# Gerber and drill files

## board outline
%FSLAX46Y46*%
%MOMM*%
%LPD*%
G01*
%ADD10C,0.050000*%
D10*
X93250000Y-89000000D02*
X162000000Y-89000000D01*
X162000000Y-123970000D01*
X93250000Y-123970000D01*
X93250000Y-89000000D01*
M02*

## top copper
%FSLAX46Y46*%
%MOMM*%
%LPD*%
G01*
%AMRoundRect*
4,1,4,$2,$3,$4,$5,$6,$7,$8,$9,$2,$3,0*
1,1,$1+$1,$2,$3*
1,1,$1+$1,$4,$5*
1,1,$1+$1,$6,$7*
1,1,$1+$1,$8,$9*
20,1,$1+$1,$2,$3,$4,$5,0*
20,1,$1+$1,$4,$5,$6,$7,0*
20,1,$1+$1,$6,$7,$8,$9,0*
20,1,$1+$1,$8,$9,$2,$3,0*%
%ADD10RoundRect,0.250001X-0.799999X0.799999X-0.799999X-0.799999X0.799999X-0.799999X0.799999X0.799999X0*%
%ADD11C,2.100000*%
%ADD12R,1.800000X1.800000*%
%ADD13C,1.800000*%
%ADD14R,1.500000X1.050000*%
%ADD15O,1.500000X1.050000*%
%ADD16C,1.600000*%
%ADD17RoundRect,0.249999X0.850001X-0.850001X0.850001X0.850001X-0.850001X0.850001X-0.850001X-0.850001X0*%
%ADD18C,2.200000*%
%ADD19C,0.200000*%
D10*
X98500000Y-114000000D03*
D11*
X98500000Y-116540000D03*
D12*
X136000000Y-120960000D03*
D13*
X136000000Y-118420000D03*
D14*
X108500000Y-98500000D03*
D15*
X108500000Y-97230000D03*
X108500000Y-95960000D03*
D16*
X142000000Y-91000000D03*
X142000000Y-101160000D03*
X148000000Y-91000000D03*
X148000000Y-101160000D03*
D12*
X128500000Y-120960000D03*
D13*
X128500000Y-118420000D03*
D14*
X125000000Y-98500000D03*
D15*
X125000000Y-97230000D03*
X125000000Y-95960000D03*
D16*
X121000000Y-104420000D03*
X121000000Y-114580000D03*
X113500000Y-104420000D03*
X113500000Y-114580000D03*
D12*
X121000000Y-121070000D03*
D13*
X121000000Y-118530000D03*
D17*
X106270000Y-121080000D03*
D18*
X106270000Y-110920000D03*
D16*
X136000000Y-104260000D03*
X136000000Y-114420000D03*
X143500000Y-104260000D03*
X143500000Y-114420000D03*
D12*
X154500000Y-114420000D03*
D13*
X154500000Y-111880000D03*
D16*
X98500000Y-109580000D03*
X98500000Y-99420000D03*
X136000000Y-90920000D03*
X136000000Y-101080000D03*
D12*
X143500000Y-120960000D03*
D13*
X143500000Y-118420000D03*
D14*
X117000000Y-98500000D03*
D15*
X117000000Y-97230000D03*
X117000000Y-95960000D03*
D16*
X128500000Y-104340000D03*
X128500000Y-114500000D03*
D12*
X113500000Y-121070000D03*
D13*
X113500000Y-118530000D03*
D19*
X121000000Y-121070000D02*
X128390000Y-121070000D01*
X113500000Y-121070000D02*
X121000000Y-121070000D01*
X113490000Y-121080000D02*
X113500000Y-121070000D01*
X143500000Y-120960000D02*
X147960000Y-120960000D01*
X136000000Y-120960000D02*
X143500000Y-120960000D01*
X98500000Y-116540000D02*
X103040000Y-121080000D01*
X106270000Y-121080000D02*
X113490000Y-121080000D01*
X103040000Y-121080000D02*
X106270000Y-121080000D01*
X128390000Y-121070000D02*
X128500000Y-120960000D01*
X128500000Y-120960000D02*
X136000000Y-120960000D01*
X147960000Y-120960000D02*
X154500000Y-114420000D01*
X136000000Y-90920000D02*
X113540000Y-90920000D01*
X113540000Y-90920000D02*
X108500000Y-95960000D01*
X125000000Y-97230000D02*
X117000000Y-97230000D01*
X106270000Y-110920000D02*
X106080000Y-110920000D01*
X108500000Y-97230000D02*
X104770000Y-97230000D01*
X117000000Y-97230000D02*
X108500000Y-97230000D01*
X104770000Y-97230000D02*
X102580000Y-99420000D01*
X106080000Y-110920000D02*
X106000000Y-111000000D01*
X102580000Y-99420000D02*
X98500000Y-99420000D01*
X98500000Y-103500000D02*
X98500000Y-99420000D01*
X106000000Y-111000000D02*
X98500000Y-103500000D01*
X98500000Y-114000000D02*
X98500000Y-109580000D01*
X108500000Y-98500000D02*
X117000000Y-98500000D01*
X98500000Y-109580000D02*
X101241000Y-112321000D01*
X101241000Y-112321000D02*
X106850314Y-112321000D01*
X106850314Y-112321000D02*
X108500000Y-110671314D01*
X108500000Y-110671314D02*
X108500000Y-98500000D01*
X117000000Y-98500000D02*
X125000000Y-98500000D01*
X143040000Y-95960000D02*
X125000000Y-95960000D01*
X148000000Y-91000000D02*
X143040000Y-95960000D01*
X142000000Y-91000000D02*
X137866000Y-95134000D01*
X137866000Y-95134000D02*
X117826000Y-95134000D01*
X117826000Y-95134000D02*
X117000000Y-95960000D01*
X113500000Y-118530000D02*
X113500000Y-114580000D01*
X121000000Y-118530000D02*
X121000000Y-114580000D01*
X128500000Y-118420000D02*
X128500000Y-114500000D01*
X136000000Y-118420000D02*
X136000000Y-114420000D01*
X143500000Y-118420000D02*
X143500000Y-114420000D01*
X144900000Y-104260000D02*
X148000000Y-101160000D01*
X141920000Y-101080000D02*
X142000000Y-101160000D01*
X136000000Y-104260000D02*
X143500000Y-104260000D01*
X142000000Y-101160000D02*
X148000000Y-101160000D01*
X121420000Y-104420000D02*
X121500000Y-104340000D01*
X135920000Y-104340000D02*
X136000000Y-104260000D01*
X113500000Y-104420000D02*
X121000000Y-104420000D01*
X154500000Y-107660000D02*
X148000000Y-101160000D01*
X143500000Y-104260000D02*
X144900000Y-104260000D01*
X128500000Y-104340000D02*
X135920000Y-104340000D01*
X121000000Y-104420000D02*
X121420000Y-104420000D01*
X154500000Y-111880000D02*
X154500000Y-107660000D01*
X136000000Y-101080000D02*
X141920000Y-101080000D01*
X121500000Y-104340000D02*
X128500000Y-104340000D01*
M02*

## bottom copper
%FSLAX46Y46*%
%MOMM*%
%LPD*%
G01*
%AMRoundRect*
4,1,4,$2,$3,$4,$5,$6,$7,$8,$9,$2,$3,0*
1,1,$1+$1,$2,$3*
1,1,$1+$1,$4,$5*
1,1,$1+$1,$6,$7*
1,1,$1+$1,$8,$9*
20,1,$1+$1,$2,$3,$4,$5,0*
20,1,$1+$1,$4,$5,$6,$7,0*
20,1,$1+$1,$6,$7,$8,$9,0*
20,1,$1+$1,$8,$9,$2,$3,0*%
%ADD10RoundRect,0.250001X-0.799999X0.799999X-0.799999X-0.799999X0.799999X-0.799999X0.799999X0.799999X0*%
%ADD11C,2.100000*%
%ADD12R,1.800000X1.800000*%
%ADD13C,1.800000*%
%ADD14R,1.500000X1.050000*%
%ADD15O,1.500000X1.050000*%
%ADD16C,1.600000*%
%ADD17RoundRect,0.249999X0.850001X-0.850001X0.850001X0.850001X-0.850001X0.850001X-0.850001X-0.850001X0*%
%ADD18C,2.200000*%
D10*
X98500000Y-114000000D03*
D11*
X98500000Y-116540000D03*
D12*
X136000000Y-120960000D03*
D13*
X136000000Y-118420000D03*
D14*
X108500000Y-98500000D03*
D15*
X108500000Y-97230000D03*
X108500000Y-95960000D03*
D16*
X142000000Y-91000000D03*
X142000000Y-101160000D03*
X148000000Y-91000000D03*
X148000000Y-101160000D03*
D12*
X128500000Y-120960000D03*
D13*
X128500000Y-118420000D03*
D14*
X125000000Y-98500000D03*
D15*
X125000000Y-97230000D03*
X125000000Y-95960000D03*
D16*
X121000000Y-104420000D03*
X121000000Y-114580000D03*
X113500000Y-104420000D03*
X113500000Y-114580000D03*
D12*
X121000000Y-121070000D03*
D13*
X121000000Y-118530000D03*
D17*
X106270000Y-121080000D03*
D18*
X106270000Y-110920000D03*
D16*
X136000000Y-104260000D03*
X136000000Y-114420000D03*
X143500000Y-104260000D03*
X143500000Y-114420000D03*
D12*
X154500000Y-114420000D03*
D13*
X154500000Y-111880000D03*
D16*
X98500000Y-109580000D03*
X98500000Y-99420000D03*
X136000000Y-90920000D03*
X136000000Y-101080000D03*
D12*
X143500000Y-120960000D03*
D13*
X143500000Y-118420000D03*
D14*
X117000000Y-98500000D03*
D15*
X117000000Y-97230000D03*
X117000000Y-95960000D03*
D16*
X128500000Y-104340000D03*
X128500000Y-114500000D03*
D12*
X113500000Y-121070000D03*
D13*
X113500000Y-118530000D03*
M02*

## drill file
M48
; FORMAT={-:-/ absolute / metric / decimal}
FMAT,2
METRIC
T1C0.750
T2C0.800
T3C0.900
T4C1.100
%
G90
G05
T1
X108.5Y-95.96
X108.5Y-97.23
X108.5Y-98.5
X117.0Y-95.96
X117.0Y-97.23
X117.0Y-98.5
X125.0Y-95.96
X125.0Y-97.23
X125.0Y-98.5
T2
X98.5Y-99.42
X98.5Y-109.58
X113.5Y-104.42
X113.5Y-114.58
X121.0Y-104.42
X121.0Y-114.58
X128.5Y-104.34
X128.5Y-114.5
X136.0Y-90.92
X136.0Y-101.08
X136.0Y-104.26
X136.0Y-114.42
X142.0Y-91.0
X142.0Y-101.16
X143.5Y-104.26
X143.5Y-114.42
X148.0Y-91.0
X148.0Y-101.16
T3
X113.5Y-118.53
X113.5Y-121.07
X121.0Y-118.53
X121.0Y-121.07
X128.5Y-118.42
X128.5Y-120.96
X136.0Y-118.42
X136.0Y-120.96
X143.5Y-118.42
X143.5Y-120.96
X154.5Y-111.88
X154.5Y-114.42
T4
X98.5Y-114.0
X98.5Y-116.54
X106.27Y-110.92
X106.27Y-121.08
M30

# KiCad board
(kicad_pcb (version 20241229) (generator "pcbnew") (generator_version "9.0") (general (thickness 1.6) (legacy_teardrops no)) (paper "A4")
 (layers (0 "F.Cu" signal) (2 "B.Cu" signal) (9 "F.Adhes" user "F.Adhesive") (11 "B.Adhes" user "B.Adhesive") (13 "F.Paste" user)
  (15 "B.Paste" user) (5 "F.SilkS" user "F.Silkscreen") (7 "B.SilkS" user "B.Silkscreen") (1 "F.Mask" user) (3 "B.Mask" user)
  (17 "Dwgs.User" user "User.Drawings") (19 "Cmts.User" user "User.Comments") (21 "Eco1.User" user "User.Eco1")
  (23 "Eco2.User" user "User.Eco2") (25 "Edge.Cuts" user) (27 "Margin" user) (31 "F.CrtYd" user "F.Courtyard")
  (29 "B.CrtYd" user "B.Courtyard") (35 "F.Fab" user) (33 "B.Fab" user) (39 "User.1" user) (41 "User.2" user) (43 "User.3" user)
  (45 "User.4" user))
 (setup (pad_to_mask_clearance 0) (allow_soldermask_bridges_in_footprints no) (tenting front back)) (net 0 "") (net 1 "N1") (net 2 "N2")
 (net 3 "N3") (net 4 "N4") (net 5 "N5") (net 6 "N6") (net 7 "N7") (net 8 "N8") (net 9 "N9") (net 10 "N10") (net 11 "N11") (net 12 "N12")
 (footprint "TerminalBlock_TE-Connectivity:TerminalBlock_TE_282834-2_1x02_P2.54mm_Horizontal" (layer "F.Cu") (at 98.5 114 -90)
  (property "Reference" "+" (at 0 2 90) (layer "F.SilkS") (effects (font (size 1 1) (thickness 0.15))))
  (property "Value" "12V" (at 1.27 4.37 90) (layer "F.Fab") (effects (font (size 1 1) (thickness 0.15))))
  (pad "1" thru_hole roundrect (at 0 0 270) (size 2.1 2.1) (drill 1.1) (layers "*.Cu" "*.Mask") (remove_unused_layers no)
   (roundrect_rratio 0.119048) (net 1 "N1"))
  (pad "2" thru_hole circle (at 2.54 0 270) (size 2.1 2.1) (drill 1.1) (layers "*.Cu" "*.Mask") (remove_unused_layers no) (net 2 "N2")))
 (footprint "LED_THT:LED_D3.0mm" (layer "F.Cu") (at 136 120.96 90)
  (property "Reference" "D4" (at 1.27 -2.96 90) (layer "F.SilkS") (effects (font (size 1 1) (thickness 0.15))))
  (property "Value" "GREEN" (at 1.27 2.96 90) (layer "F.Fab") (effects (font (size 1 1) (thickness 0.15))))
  (pad "1" thru_hole rect (at 0 0 90) (size 1.8 1.8) (drill 0.9) (layers "*.Cu" "*.Mask") (remove_unused_layers no) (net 2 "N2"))
  (pad "2" thru_hole circle (at 2.54 0 90) (size 1.8 1.8) (drill 0.9) (layers "*.Cu" "*.Mask") (remove_unused_layers no) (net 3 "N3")))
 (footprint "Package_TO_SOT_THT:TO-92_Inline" (layer "F.Cu") (at 108.5 98.5 90)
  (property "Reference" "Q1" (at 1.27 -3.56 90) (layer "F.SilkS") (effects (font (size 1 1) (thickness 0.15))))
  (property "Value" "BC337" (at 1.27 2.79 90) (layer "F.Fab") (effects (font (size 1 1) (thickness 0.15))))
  (pad "1" thru_hole rect (at 0 0 90) (size 1.05 1.5) (drill 0.75) (layers "*.Cu" "*.Mask") (remove_unused_layers no) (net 1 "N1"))
  (pad "2" thru_hole oval (at 1.27 0 90) (size 1.05 1.5) (drill 0.75) (layers "*.Cu" "*.Mask") (remove_unused_layers no) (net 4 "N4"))
  (pad "3" thru_hole oval (at 2.54 0 90) (size 1.05 1.5) (drill 0.75) (layers "*.Cu" "*.Mask") (remove_unused_layers no) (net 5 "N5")))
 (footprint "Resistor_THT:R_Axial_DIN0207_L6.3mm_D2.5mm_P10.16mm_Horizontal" (layer "F.Cu") (at 142 91 -90)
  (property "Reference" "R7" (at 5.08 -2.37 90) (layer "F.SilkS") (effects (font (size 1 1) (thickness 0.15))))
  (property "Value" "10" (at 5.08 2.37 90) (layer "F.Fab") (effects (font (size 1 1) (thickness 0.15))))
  (pad "1" thru_hole circle (at 0 0 270) (size 1.6 1.6) (drill 0.8) (layers "*.Cu" "*.Mask") (remove_unused_layers no) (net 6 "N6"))
  (pad "2" thru_hole circle (at 10.16 0 270) (size 1.6 1.6) (drill 0.8) (layers "*.Cu" "*.Mask") (remove_unused_layers no) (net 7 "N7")))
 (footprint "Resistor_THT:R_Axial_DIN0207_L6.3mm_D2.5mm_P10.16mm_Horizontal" (layer "F.Cu") (at 148 91 -90)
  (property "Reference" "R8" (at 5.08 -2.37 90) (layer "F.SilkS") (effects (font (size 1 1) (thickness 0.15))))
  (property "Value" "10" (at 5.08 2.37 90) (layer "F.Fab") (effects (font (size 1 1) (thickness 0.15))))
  (pad "1" thru_hole circle (at 0 0 270) (size 1.6 1.6) (drill 0.8) (layers "*.Cu" "*.Mask") (remove_unused_layers no) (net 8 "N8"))
  (pad "2" thru_hole circle (at 10.16 0 270) (size 1.6 1.6) (drill 0.8) (layers "*.Cu" "*.Mask") (remove_unused_layers no) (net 7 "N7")))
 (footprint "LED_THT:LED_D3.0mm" (layer "F.Cu") (at 128.5 120.96 90)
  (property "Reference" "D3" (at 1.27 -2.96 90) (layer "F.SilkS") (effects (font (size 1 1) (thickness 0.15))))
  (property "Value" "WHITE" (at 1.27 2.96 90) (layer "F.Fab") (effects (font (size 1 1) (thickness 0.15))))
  (pad "1" thru_hole rect (at 0 0 90) (size 1.8 1.8) (drill 0.9) (layers "*.Cu" "*.Mask") (remove_unused_layers no) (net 2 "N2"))
  (pad "2" thru_hole circle (at 2.54 0 90) (size 1.8 1.8) (drill 0.9) (layers "*.Cu" "*.Mask") (remove_unused_layers no) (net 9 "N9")))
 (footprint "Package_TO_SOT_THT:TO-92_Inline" (layer "F.Cu") (at 125 98.5 90)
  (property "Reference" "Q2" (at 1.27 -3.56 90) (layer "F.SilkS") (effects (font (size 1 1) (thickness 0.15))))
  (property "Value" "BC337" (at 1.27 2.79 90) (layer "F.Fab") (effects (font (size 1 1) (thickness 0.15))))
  (pad "1" thru_hole rect (at 0 0 90) (size 1.05 1.5) (drill 0.75) (layers "*.Cu" "*.Mask") (remove_unused_layers no) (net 1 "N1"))
  (pad "2" thru_hole oval (at 1.27 0 90) (size 1.05 1.5) (drill 0.75) (layers "*.Cu" "*.Mask") (remove_unused_layers no) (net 4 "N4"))
  (pad "3" thru_hole oval (at 2.54 0 90) (size 1.05 1.5) (drill 0.75) (layers "*.Cu" "*.Mask") (remove_unused_layers no) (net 8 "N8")))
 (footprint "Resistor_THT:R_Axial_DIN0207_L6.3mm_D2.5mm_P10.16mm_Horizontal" (layer "F.Cu") (at 121 104.42 -90)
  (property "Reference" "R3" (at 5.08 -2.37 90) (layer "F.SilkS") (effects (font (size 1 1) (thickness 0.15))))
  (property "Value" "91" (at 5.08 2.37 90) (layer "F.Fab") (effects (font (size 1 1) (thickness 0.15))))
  (pad "1" thru_hole circle (at 0 0 270) (size 1.6 1.6) (drill 0.8) (layers "*.Cu" "*.Mask") (remove_unused_layers no) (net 7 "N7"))
  (pad "2" thru_hole circle (at 10.16 0 270) (size 1.6 1.6) (drill 0.8) (layers "*.Cu" "*.Mask") (remove_unused_layers no) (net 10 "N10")))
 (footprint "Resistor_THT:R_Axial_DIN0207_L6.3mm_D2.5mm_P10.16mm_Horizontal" (layer "F.Cu") (at 113.5 104.42 -90)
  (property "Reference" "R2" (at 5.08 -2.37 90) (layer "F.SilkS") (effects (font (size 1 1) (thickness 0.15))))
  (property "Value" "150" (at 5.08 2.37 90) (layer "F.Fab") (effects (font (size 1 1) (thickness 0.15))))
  (pad "1" thru_hole circle (at 0 0 270) (size 1.6 1.6) (drill 0.8) (layers "*.Cu" "*.Mask") (remove_unused_layers no) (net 7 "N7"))
  (pad "2" thru_hole circle (at 10.16 0 270) (size 1.6 1.6) (drill 0.8) (layers "*.Cu" "*.Mask") (remove_unused_layers no) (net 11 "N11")))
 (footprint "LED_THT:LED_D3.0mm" (layer "F.Cu") (at 121 121.07 90)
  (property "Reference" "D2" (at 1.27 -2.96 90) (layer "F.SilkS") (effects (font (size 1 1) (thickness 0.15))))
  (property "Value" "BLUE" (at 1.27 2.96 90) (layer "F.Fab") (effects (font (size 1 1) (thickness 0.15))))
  (pad "1" thru_hole rect (at 0 0 90) (size 1.8 1.8) (drill 0.9) (layers "*.Cu" "*.Mask") (remove_unused_layers no) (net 2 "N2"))
  (pad "2" thru_hole circle (at 2.54 0 90) (size 1.8 1.8) (drill 0.9) (layers "*.Cu" "*.Mask") (remove_unused_layers no) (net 10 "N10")))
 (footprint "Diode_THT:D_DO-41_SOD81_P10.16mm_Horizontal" (layer "F.Cu") (at 106.27 121.08 90)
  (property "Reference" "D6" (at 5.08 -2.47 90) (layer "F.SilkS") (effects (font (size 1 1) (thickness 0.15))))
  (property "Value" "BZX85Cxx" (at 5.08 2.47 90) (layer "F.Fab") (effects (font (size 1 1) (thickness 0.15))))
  (pad "1" thru_hole roundrect (at 0 0 90) (size 2.2 2.2) (drill 1.1) (layers "*.Cu" "*.Mask") (remove_unused_layers no)
   (roundrect_rratio 0.113636) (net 2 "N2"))
  (pad "2" thru_hole circle (at 10.16 0 90) (size 2.2 2.2) (drill 1.1) (layers "*.Cu" "*.Mask") (remove_unused_layers no) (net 4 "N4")))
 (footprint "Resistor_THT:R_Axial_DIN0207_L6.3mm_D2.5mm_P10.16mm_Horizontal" (layer "F.Cu") (at 136 104.26 -90)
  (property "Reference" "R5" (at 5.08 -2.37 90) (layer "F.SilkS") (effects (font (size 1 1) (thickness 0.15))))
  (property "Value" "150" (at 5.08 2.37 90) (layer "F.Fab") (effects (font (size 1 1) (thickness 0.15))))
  (pad "1" thru_hole circle (at 0 0 270) (size 1.6 1.6) (drill 0.8) (layers "*.Cu" "*.Mask") (remove_unused_layers no) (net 7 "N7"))
  (pad "2" thru_hole circle (at 10.16 0 270) (size 1.6 1.6) (drill 0.8) (layers "*.Cu" "*.Mask") (remove_unused_layers no) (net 3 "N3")))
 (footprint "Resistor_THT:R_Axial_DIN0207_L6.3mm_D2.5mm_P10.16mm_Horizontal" (layer "F.Cu") (at 143.5 104.26 -90)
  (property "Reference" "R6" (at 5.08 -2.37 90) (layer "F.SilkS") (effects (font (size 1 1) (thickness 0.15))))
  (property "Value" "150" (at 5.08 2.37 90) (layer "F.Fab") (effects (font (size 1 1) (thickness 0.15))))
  (pad "1" thru_hole circle (at 0 0 270) (size 1.6 1.6) (drill 0.8) (layers "*.Cu" "*.Mask") (remove_unused_layers no) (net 7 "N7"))
  (pad "2" thru_hole circle (at 10.16 0 270) (size 1.6 1.6) (drill 0.8) (layers "*.Cu" "*.Mask") (remove_unused_layers no) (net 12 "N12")))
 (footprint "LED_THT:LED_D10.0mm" (layer "F.Cu") (at 154.5 114.42 90)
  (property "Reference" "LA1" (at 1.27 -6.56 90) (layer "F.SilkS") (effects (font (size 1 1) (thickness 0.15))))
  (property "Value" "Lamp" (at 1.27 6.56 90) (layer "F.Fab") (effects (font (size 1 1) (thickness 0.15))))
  (pad "1" thru_hole rect (at 0 0 90) (size 1.8 1.8) (drill 0.9) (layers "*.Cu" "*.Mask") (remove_unused_layers no) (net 2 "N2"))
  (pad "2" thru_hole circle (at 2.54 0 90) (size 1.8 1.8) (drill 0.9) (layers "*.Cu" "*.Mask") (remove_unused_layers no) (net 7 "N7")))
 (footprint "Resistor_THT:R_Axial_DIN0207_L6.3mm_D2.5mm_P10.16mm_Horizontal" (layer "F.Cu") (at 98.5 109.58 90)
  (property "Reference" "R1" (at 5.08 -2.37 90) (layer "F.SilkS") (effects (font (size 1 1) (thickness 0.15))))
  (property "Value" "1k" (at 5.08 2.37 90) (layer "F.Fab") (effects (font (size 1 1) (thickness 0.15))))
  (pad "1" thru_hole circle (at 0 0 90) (size 1.6 1.6) (drill 0.8) (layers "*.Cu" "*.Mask") (remove_unused_layers no) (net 1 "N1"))
  (pad "2" thru_hole circle (at 10.16 0 90) (size 1.6 1.6) (drill 0.8) (layers "*.Cu" "*.Mask") (remove_unused_layers no) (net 4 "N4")))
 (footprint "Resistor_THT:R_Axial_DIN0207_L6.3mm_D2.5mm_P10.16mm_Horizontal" (layer "F.Cu") (at 136 90.92 -90)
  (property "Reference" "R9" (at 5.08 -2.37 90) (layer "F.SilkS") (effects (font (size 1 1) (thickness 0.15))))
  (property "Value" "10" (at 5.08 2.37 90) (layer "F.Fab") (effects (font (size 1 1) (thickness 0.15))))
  (pad "1" thru_hole circle (at 0 0 270) (size 1.6 1.6) (drill 0.8) (layers "*.Cu" "*.Mask") (remove_unused_layers no) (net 5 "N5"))
  (pad "2" thru_hole circle (at 10.16 0 270) (size 1.6 1.6) (drill 0.8) (layers "*.Cu" "*.Mask") (remove_unused_layers no) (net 7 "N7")))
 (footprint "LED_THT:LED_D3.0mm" (layer "F.Cu") (at 143.5 120.96 90)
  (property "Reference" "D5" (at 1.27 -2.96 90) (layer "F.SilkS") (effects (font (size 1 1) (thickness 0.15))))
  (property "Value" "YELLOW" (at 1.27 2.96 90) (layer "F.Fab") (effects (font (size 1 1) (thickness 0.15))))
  (pad "1" thru_hole rect (at 0 0 90) (size 1.8 1.8) (drill 0.9) (layers "*.Cu" "*.Mask") (remove_unused_layers no) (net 2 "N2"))
  (pad "2" thru_hole circle (at 2.54 0 90) (size 1.8 1.8) (drill 0.9) (layers "*.Cu" "*.Mask") (remove_unused_layers no) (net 12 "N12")))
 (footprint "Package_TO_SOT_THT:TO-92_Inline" (layer "F.Cu") (at 117 98.5 90)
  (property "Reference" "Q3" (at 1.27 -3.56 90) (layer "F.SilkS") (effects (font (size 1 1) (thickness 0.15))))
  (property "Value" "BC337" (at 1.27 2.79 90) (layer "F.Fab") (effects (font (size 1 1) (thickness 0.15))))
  (pad "1" thru_hole rect (at 0 0 90) (size 1.05 1.5) (drill 0.75) (layers "*.Cu" "*.Mask") (remove_unused_layers no) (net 1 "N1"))
  (pad "2" thru_hole oval (at 1.27 0 90) (size 1.05 1.5) (drill 0.75) (layers "*.Cu" "*.Mask") (remove_unused_layers no) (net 4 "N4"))
  (pad "3" thru_hole oval (at 2.54 0 90) (size 1.05 1.5) (drill 0.75) (layers "*.Cu" "*.Mask") (remove_unused_layers no) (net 6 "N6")))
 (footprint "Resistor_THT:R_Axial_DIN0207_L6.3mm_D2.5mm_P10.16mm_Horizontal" (layer "F.Cu") (at 128.5 104.34 -90)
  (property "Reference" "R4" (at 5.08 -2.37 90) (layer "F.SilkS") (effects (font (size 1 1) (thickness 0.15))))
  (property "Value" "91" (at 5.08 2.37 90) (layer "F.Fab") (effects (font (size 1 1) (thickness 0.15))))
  (pad "1" thru_hole circle (at 0 0 270) (size 1.6 1.6) (drill 0.8) (layers "*.Cu" "*.Mask") (remove_unused_layers no) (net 7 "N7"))
  (pad "2" thru_hole circle (at 10.16 0 270) (size 1.6 1.6) (drill 0.8) (layers "*.Cu" "*.Mask") (remove_unused_layers no) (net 9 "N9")))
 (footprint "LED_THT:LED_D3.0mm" (layer "F.Cu") (at 113.5 121.07 90)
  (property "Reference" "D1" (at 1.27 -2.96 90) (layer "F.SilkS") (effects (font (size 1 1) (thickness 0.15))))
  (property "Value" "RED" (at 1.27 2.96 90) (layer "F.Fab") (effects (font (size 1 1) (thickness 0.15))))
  (pad "1" thru_hole rect (at 0 0 90) (size 1.8 1.8) (drill 0.9) (layers "*.Cu" "*.Mask") (remove_unused_layers no) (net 2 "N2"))
  (pad "2" thru_hole circle (at 2.54 0 90) (size 1.8 1.8) (drill 0.9) (layers "*.Cu" "*.Mask") (remove_unused_layers no) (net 11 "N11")))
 (gr_rect (start 93.25 89) (end 162 123.97) (stroke (width 0.05) (type default)) (fill no) (layer "Edge.Cuts"))
 (segment (start 121 121.07) (end 128.39 121.07) (width 0.2) (layer "F.Cu") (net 2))
 (segment (start 113.5 121.07) (end 121 121.07) (width 0.2) (layer "F.Cu") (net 2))
 (segment (start 113.49 121.08) (end 113.5 121.07) (width 0.2) (layer "F.Cu") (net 2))
 (segment (start 143.5 120.96) (end 147.96 120.96) (width 0.2) (layer "F.Cu") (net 2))
 (segment (start 136 120.96) (end 143.5 120.96) (width 0.2) (layer "F.Cu") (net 2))
 (segment (start 98.5 116.54) (end 103.04 121.08) (width 0.2) (layer "F.Cu") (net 2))
 (segment (start 106.27 121.08) (end 113.49 121.08) (width 0.2) (layer "F.Cu") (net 2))
 (segment (start 103.04 121.08) (end 106.27 121.08) (width 0.2) (layer "F.Cu") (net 2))
 (segment (start 128.39 121.07) (end 128.5 120.96) (width 0.2) (layer "F.Cu") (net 2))
 (segment (start 128.5 120.96) (end 136 120.96) (width 0.2) (layer "F.Cu") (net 2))
 (segment (start 147.96 120.96) (end 154.5 114.42) (width 0.2) (layer "F.Cu") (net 2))
 (segment (start 136 90.92) (end 113.54 90.92) (width 0.2) (layer "F.Cu") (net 5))
 (segment (start 113.54 90.92) (end 108.5 95.96) (width 0.2) (layer "F.Cu") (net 5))
 (segment (start 125 97.23) (end 117 97.23) (width 0.2) (layer "F.Cu") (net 4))
 (segment (start 106.27 110.92) (end 106.08 110.92) (width 0.2) (layer "F.Cu") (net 4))
 (segment (start 108.5 97.23) (end 104.77 97.23) (width 0.2) (layer "F.Cu") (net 4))
 (segment (start 117 97.23) (end 108.5 97.23) (width 0.2) (layer "F.Cu") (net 4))
 (segment (start 104.77 97.23) (end 102.58 99.42) (width 0.2) (layer "F.Cu") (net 4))
 (segment (start 106.08 110.92) (end 106 111) (width 0.2) (layer "F.Cu") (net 4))
 (segment (start 102.58 99.42) (end 98.5 99.42) (width 0.2) (layer "F.Cu") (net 4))
 (segment (start 98.5 103.5) (end 98.5 99.42) (width 0.2) (layer "F.Cu") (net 4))
 (segment (start 106 111) (end 98.5 103.5) (width 0.2) (layer "F.Cu") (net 4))
 (segment (start 98.5 114) (end 98.5 109.58) (width 0.2) (layer "F.Cu") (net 1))
 (segment (start 108.5 98.5) (end 117 98.5) (width 0.2) (layer "F.Cu") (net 1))
 (segment (start 98.5 109.58) (end 101.241 112.321) (width 0.2) (layer "F.Cu") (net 1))
 (segment (start 101.241 112.321) (end 106.850314 112.321) (width 0.2) (layer "F.Cu") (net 1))
 (segment (start 106.850314 112.321) (end 108.5 110.671314) (width 0.2) (layer "F.Cu") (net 1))
 (segment (start 108.5 110.671314) (end 108.5 98.5) (width 0.2) (layer "F.Cu") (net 1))
 (segment (start 117 98.5) (end 125 98.5) (width 0.2) (layer "F.Cu") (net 1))
 (segment (start 143.04 95.96) (end 125 95.96) (width 0.2) (layer "F.Cu") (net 8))
 (segment (start 148 91) (end 143.04 95.96) (width 0.2) (layer "F.Cu") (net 8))
 (segment (start 142 91) (end 137.866 95.134) (width 0.2) (layer "F.Cu") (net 6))
 (segment (start 137.866 95.134) (end 117.826 95.134) (width 0.2) (layer "F.Cu") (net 6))
 (segment (start 117.826 95.134) (end 117 95.96) (width 0.2) (layer "F.Cu") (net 6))
 (segment (start 113.5 118.53) (end 113.5 114.58) (width 0.2) (layer "F.Cu") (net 11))
 (segment (start 121 118.53) (end 121 114.58) (width 0.2) (layer "F.Cu") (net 10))
 (segment (start 128.5 118.42) (end 128.5 114.5) (width 0.2) (layer "F.Cu") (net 9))
 (segment (start 136 118.42) (end 136 114.42) (width 0.2) (layer "F.Cu") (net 3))
 (segment (start 143.5 118.42) (end 143.5 114.42) (width 0.2) (layer "F.Cu") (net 12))
 (segment (start 144.9 104.26) (end 148 101.16) (width 0.2) (layer "F.Cu") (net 7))
 (segment (start 141.92 101.08) (end 142 101.16) (width 0.2) (layer "F.Cu") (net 7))
 (segment (start 136 104.26) (end 143.5 104.26) (width 0.2) (layer "F.Cu") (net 7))
 (segment (start 142 101.16) (end 148 101.16) (width 0.2) (layer "F.Cu") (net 7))
 (segment (start 121.42 104.42) (end 121.5 104.34) (width 0.2) (layer "F.Cu") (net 7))
 (segment (start 135.92 104.34) (end 136 104.26) (width 0.2) (layer "F.Cu") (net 7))
 (segment (start 113.5 104.42) (end 121 104.42) (width 0.2) (layer "F.Cu") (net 7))
 (segment (start 154.5 107.66) (end 148 101.16) (width 0.2) (layer "F.Cu") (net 7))
 (segment (start 143.5 104.26) (end 144.9 104.26) (width 0.2) (layer "F.Cu") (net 7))
 (segment (start 128.5 104.34) (end 135.92 104.34) (width 0.2) (layer "F.Cu") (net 7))
 (segment (start 121 104.42) (end 121.42 104.42) (width 0.2) (layer "F.Cu") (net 7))
 (segment (start 154.5 111.88) (end 154.5 107.66) (width 0.2) (layer "F.Cu") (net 7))
 (segment (start 136 101.08) (end 141.92 101.08) (width 0.2) (layer "F.Cu") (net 7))
 (segment (start 121.5 104.34) (end 128.5 104.34) (width 0.2) (layer "F.Cu") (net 7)))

